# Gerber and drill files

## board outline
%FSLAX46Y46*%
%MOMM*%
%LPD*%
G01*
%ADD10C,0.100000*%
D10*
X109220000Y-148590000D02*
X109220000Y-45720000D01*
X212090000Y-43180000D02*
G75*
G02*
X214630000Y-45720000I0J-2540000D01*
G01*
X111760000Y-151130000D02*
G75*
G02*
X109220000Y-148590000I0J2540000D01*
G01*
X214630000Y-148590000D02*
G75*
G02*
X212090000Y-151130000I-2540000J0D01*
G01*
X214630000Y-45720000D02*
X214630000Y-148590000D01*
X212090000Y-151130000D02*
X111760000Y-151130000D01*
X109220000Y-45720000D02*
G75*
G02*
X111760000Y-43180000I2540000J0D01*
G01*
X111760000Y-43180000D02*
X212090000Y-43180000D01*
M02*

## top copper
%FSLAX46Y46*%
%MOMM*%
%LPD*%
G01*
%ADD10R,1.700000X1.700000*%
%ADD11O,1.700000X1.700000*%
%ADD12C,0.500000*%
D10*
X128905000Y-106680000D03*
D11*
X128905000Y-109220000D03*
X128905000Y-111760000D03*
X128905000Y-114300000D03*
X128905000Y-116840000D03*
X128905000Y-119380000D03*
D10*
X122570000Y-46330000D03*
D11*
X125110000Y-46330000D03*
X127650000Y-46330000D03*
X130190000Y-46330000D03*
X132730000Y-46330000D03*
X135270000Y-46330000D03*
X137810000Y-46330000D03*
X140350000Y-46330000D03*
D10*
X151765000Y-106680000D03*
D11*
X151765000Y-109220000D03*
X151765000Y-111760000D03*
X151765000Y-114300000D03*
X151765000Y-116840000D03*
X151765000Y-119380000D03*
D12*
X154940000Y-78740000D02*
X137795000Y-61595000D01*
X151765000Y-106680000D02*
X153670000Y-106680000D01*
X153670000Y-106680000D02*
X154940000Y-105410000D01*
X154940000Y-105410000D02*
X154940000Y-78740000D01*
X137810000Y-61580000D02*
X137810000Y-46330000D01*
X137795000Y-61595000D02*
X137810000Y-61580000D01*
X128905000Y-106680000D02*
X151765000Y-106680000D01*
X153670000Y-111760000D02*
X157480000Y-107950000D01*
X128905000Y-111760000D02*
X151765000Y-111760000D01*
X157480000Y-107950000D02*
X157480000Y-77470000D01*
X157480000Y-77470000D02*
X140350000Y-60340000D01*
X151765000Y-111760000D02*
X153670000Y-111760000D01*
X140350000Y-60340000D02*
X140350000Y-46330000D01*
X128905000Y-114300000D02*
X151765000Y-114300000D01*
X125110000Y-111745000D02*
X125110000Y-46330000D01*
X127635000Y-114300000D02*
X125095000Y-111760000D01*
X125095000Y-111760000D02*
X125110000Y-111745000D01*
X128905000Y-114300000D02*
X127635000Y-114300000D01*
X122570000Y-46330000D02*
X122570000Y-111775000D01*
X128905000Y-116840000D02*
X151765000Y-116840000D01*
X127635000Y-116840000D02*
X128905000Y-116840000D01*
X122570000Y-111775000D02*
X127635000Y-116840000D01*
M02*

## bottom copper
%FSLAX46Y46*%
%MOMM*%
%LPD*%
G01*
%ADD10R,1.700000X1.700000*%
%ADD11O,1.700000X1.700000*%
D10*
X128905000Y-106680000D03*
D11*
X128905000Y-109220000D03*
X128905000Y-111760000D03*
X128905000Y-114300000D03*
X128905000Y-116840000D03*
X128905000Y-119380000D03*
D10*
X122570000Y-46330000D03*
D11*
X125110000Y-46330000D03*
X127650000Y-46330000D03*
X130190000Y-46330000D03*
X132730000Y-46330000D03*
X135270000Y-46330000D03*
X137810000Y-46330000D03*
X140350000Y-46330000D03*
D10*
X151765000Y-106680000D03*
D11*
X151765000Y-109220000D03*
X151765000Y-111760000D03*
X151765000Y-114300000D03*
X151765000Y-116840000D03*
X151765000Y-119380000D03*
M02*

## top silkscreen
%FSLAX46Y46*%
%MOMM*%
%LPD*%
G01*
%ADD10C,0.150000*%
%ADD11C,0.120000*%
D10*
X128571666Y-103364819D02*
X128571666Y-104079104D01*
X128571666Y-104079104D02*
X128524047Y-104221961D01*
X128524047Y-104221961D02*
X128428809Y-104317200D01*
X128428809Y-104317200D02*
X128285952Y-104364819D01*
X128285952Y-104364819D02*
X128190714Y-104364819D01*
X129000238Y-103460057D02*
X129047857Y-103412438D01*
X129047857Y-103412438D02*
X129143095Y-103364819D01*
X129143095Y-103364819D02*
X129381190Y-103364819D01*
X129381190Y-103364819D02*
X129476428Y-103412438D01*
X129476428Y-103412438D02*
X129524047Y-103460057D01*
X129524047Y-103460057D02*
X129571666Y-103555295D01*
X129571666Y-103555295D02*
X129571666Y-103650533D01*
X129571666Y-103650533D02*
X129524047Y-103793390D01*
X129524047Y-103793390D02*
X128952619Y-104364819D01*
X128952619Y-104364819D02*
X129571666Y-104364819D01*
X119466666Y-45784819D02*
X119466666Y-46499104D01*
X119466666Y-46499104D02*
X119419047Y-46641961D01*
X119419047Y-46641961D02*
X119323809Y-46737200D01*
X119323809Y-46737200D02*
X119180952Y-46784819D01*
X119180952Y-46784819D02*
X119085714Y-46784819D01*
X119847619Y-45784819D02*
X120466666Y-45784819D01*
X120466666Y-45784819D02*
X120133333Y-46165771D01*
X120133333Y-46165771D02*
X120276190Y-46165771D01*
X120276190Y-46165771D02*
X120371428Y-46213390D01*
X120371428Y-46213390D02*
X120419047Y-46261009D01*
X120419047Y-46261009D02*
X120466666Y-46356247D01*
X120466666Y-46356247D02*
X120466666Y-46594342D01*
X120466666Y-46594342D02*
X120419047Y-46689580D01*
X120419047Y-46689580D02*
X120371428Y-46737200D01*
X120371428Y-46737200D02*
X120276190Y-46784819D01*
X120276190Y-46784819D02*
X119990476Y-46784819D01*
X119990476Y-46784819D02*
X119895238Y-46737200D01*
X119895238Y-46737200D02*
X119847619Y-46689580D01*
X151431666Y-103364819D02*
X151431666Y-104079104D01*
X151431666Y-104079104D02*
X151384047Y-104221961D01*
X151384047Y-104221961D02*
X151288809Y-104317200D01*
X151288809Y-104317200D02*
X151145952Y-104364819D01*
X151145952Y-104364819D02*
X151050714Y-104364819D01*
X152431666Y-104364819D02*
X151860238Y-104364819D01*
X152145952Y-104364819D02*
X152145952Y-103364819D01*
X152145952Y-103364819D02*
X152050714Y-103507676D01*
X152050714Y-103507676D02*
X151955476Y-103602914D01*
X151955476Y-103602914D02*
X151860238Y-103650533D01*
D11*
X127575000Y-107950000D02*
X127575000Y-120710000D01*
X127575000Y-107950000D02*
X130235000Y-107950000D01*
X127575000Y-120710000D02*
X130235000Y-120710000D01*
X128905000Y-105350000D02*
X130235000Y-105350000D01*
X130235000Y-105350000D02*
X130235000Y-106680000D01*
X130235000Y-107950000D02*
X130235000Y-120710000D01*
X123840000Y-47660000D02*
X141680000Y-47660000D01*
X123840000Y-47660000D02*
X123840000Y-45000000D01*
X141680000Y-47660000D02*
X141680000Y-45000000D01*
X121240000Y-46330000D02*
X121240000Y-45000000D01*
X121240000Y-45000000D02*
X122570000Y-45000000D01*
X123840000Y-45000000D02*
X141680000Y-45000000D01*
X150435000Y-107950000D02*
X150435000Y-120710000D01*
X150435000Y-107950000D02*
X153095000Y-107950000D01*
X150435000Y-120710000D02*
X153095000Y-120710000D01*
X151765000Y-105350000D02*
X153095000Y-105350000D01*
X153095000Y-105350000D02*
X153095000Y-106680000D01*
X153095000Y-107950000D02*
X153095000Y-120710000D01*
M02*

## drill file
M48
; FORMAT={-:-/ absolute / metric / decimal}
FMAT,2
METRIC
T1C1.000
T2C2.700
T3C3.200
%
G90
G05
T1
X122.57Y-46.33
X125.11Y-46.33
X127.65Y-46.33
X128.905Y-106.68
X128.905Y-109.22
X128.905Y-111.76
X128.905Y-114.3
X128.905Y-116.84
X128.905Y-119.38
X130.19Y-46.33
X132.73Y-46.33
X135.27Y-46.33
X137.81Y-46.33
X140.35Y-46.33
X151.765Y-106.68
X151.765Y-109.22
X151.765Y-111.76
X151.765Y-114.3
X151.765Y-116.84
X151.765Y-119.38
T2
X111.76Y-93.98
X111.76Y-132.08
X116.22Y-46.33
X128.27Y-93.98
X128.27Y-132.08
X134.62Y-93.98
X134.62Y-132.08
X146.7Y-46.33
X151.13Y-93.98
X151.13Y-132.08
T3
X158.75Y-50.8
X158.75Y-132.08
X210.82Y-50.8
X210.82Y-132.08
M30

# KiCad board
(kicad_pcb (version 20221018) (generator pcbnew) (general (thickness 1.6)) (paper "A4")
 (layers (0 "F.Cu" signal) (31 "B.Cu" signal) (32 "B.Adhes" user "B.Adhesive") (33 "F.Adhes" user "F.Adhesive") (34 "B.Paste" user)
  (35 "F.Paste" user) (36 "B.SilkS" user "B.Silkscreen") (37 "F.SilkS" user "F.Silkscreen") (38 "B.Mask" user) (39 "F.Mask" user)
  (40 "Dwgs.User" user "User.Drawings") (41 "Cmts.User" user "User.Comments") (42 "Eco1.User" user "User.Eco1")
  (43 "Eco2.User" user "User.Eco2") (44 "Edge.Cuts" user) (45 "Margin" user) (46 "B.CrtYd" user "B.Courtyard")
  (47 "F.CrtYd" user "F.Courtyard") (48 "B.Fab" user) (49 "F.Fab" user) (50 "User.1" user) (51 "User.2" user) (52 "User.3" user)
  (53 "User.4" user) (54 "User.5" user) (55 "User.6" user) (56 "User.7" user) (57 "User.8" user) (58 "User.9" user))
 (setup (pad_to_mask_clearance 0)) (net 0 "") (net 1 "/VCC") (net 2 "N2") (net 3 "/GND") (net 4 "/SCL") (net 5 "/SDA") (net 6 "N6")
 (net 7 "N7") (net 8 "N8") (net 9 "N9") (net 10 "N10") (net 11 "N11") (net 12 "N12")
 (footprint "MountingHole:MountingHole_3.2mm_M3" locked (layer "F.Cu") (at 158.75 132.08)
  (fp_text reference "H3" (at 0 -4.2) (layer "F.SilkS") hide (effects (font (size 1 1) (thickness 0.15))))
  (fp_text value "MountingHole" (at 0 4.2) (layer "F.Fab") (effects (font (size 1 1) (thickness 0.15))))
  (pad "" np_thru_hole circle locked (at 0 0) (size 3.2 3.2) (drill 3.2) (layers "*.Cu" "*.Mask")))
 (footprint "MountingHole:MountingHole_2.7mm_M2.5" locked (layer "F.Cu") (at 146.7 46.33)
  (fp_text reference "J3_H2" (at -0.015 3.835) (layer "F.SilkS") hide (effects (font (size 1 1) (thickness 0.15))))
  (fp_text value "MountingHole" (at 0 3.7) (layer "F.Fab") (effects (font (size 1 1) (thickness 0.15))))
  (pad "" np_thru_hole circle locked (at 0 0) (size 2.7 2.7) (drill 2.7) (layers "*.Cu" "*.Mask")))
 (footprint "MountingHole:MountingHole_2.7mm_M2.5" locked (layer "F.Cu") (at 128.27 93.98)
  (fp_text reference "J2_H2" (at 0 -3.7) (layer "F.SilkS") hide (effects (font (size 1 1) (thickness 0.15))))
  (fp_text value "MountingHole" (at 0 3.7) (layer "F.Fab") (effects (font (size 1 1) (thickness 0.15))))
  (pad "" np_thru_hole circle locked (at 0 0) (size 2.7 2.7) (drill 2.7) (layers "*.Cu" "*.Mask")))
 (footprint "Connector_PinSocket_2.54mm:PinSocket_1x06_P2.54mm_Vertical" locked (layer "F.Cu") (at 128.905 106.68)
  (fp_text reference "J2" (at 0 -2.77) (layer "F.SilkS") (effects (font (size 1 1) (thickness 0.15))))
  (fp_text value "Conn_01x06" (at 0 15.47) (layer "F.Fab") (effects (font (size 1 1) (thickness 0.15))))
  (fp_line (start -1.33 1.27) (end -1.33 14.03) (stroke (width 0.12) (type solid)) (layer "F.SilkS"))
  (fp_line (start -1.33 1.27) (end 1.33 1.27) (stroke (width 0.12) (type solid)) (layer "F.SilkS"))
  (fp_line (start -1.33 14.03) (end 1.33 14.03) (stroke (width 0.12) (type solid)) (layer "F.SilkS"))
  (fp_line (start 0 -1.33) (end 1.33 -1.33) (stroke (width 0.12) (type solid)) (layer "F.SilkS"))
  (fp_line (start 1.33 -1.33) (end 1.33 0) (stroke (width 0.12) (type solid)) (layer "F.SilkS"))
  (fp_line (start 1.33 1.27) (end 1.33 14.03) (stroke (width 0.12) (type solid)) (layer "F.SilkS"))
  (pad "1" thru_hole rect locked (at 0 0) (size 1.7 1.7) (drill 1) (layers "*.Cu" "*.Mask") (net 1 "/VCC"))
  (pad "2" thru_hole oval locked (at 0 2.54) (size 1.7 1.7) (drill 1) (layers "*.Cu" "*.Mask") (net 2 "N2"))
  (pad "3" thru_hole oval locked (at 0 5.08) (size 1.7 1.7) (drill 1) (layers "*.Cu" "*.Mask") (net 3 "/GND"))
  (pad "4" thru_hole oval locked (at 0 7.62) (size 1.7 1.7) (drill 1) (layers "*.Cu" "*.Mask") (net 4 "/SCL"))
  (pad "5" thru_hole oval locked (at 0 10.16) (size 1.7 1.7) (drill 1) (layers "*.Cu" "*.Mask") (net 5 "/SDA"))
  (pad "6" thru_hole oval locked (at 0 12.7) (size 1.7 1.7) (drill 1) (layers "*.Cu" "*.Mask") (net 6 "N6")))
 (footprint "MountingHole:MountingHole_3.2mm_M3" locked (layer "F.Cu") (at 158.75 50.8)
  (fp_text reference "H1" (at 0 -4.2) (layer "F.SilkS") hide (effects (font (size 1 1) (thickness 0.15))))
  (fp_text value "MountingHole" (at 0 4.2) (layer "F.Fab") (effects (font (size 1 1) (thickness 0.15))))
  (pad "" np_thru_hole circle locked (at 0 0) (size 3.2 3.2) (drill 3.2) (layers "*.Cu" "*.Mask")))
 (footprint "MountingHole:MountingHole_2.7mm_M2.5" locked (layer "F.Cu") (at 134.62 132.08)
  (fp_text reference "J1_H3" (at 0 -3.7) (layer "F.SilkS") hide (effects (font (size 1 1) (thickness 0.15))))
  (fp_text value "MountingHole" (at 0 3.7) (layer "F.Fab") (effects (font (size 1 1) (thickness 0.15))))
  (pad "" np_thru_hole circle locked (at 0 0) (size 2.7 2.7) (drill 2.7) (layers "*.Cu" "*.Mask")))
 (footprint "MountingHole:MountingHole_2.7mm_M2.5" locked (layer "F.Cu") (at 116.22 46.33)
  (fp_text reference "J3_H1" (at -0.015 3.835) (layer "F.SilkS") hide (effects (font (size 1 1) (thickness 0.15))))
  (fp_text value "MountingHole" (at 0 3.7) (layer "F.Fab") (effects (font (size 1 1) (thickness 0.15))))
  (pad "" np_thru_hole circle locked (at 0 0) (size 2.7 2.7) (drill 2.7) (layers "*.Cu" "*.Mask")))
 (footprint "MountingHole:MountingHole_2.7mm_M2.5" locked (layer "F.Cu") (at 151.13 132.08)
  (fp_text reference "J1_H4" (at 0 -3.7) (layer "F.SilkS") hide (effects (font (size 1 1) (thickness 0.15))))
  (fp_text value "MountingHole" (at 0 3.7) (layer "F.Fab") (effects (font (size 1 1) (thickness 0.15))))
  (pad "" np_thru_hole circle locked (at 0 0) (size 2.7 2.7) (drill 2.7) (layers "*.Cu" "*.Mask")))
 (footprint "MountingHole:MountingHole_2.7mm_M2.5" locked (layer "F.Cu") (at 134.62 93.98)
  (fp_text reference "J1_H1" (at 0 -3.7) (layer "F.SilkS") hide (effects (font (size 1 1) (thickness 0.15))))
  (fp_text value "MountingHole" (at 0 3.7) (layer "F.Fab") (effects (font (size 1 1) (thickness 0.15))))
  (pad "" np_thru_hole circle locked (at 0 0) (size 2.7 2.7) (drill 2.7) (layers "*.Cu" "*.Mask")))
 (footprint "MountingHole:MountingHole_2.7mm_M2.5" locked (layer "F.Cu") (at 111.76 132.08)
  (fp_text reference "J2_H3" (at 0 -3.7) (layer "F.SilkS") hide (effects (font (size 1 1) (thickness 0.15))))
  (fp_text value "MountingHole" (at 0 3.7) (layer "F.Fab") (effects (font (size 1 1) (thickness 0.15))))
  (pad "" np_thru_hole circle locked (at 0 0) (size 2.7 2.7) (drill 2.7) (layers "*.Cu" "*.Mask")))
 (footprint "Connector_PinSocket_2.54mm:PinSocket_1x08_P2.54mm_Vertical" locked (layer "F.Cu") (at 122.57 46.33 90)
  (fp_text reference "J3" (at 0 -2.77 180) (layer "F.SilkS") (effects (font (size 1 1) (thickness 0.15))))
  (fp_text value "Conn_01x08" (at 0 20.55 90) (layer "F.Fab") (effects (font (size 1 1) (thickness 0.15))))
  (fp_line (start -1.33 1.27) (end -1.33 19.11) (stroke (width 0.12) (type solid)) (layer "F.SilkS"))
  (fp_line (start -1.33 1.27) (end 1.33 1.27) (stroke (width 0.12) (type solid)) (layer "F.SilkS"))
  (fp_line (start -1.33 19.11) (end 1.33 19.11) (stroke (width 0.12) (type solid)) (layer "F.SilkS"))
  (fp_line (start 0 -1.33) (end 1.33 -1.33) (stroke (width 0.12) (type solid)) (layer "F.SilkS"))
  (fp_line (start 1.33 -1.33) (end 1.33 0) (stroke (width 0.12) (type solid)) (layer "F.SilkS"))
  (fp_line (start 1.33 1.27) (end 1.33 19.11) (stroke (width 0.12) (type solid)) (layer "F.SilkS"))
  (pad "1" thru_hole rect locked (at 0 0 90) (size 1.7 1.7) (drill 1) (layers "*.Cu" "*.Mask") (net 5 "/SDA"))
  (pad "2" thru_hole oval locked (at 0 2.54 90) (size 1.7 1.7) (drill 1) (layers "*.Cu" "*.Mask") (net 4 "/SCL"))
  (pad "3" thru_hole oval locked (at 0 5.08 90) (size 1.7 1.7) (drill 1) (layers "*.Cu" "*.Mask") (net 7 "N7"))
  (pad "4" thru_hole oval locked (at 0 7.62 90) (size 1.7 1.7) (drill 1) (layers "*.Cu" "*.Mask") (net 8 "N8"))
  (pad "5" thru_hole oval locked (at 0 10.16 90) (size 1.7 1.7) (drill 1) (layers "*.Cu" "*.Mask") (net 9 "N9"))
  (pad "6" thru_hole oval locked (at 0 12.7 90) (size 1.7 1.7) (drill 1) (layers "*.Cu" "*.Mask") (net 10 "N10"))
  (pad "7" thru_hole oval locked (at 0 15.24 90) (size 1.7 1.7) (drill 1) (layers "*.Cu" "*.Mask") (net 1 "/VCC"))
  (pad "8" thru_hole oval locked (at 0 17.78 90) (size 1.7 1.7) (drill 1) (layers "*.Cu" "*.Mask") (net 3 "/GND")))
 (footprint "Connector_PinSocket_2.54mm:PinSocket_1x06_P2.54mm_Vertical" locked (layer "F.Cu") (at 151.765 106.68)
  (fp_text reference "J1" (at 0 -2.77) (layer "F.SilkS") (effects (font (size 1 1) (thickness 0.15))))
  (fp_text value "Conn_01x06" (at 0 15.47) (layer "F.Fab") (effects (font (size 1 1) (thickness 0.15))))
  (fp_line (start -1.33 1.27) (end -1.33 14.03) (stroke (width 0.12) (type solid)) (layer "F.SilkS"))
  (fp_line (start -1.33 1.27) (end 1.33 1.27) (stroke (width 0.12) (type solid)) (layer "F.SilkS"))
  (fp_line (start -1.33 14.03) (end 1.33 14.03) (stroke (width 0.12) (type solid)) (layer "F.SilkS"))
  (fp_line (start 0 -1.33) (end 1.33 -1.33) (stroke (width 0.12) (type solid)) (layer "F.SilkS"))
  (fp_line (start 1.33 -1.33) (end 1.33 0) (stroke (width 0.12) (type solid)) (layer "F.SilkS"))
  (fp_line (start 1.33 1.27) (end 1.33 14.03) (stroke (width 0.12) (type solid)) (layer "F.SilkS"))
  (pad "1" thru_hole rect locked (at 0 0) (size 1.7 1.7) (drill 1) (layers "*.Cu" "*.Mask") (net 1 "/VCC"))
  (pad "2" thru_hole oval locked (at 0 2.54) (size 1.7 1.7) (drill 1) (layers "*.Cu" "*.Mask") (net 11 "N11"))
  (pad "3" thru_hole oval locked (at 0 5.08) (size 1.7 1.7) (drill 1) (layers "*.Cu" "*.Mask") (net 3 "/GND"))
  (pad "4" thru_hole oval locked (at 0 7.62) (size 1.7 1.7) (drill 1) (layers "*.Cu" "*.Mask") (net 4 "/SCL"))
  (pad "5" thru_hole oval locked (at 0 10.16) (size 1.7 1.7) (drill 1) (layers "*.Cu" "*.Mask") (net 5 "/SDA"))
  (pad "6" thru_hole oval locked (at 0 12.7) (size 1.7 1.7) (drill 1) (layers "*.Cu" "*.Mask") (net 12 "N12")))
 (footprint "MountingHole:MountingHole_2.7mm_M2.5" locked (layer "F.Cu") (at 151.13 93.98)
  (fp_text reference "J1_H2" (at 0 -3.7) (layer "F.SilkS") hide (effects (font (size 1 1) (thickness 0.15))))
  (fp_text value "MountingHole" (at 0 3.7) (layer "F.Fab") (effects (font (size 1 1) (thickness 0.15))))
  (pad "" np_thru_hole circle locked (at 0 0) (size 2.7 2.7) (drill 2.7) (layers "*.Cu" "*.Mask")))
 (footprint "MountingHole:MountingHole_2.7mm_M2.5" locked (layer "F.Cu") (at 128.27 132.08)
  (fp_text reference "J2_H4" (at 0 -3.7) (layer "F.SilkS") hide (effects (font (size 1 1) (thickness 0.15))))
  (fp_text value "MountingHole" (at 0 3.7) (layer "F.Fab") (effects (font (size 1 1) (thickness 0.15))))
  (pad "" np_thru_hole circle locked (at 0 0) (size 2.7 2.7) (drill 2.7) (layers "*.Cu" "*.Mask")))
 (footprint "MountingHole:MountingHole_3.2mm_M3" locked (layer "F.Cu") (at 210.82 50.8)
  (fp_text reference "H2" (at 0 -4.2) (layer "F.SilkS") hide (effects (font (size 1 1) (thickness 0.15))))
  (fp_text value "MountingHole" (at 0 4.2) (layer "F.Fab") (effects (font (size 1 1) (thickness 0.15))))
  (pad "" np_thru_hole circle locked (at 0 0) (size 3.2 3.2) (drill 3.2) (layers "*.Cu" "*.Mask")))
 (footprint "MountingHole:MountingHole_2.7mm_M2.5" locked (layer "F.Cu") (at 111.76 93.98)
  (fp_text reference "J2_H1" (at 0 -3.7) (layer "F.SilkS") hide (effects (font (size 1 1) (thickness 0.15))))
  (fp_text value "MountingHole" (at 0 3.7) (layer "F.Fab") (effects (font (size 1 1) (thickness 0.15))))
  (pad "" np_thru_hole circle locked (at 0 0) (size 2.7 2.7) (drill 2.7) (layers "*.Cu" "*.Mask")))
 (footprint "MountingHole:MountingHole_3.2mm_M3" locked (layer "F.Cu") (at 210.82 132.08)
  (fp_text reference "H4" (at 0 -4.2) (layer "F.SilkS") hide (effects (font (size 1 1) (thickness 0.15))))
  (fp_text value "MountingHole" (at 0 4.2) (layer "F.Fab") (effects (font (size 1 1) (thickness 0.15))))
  (pad "" np_thru_hole circle locked (at 0 0) (size 3.2 3.2) (drill 3.2) (layers "*.Cu" "*.Mask")))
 (gr_line (start 109.22 148.59) (end 109.22 45.72) (stroke (width 0.1) (type default)) (layer "Edge.Cuts"))
 (gr_arc (start 212.09 43.18) (mid 213.886051 43.923949) (end 214.63 45.72) (stroke (width 0.1) (type default)) (layer "Edge.Cuts"))
 (gr_arc (start 111.76 151.13) (mid 109.963949 150.386051) (end 109.22 148.59) (stroke (width 0.1) (type default)) (layer "Edge.Cuts"))
 (gr_arc (start 214.63 148.59) (mid 213.886051 150.386051) (end 212.09 151.13) (stroke (width 0.1) (type default)) (layer "Edge.Cuts"))
 (gr_line (start 214.63 45.72) (end 214.63 148.59) (stroke (width 0.1) (type default)) (layer "Edge.Cuts"))
 (gr_line (start 212.09 151.13) (end 111.76 151.13) (stroke (width 0.1) (type default)) (layer "Edge.Cuts"))
 (gr_arc (start 109.22 45.72) (mid 109.963949 43.923949) (end 111.76 43.18) (stroke (width 0.1) (type default)) (layer "Edge.Cuts"))
 (gr_line (start 111.76 43.18) (end 212.09 43.18) (stroke (width 0.1) (type default)) (layer "Edge.Cuts"))
 (segment (start 154.94 78.74) (end 137.795 61.595) (width 0.5) (layer "F.Cu") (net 1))
 (segment (start 151.765 106.68) (end 153.67 106.68) (width 0.5) (layer "F.Cu") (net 1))
 (segment (start 153.67 106.68) (end 154.94 105.41) (width 0.5) (layer "F.Cu") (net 1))
 (segment (start 154.94 105.41) (end 154.94 78.74) (width 0.5) (layer "F.Cu") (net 1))
 (segment (start 137.81 61.58) (end 137.81 46.33) (width 0.5) (layer "F.Cu") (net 1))
 (segment (start 137.795 61.595) (end 137.81 61.58) (width 0.5) (layer "F.Cu") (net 1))
 (segment (start 128.905 106.68) (end 151.765 106.68) (width 0.5) (layer "F.Cu") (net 1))
 (segment (start 153.67 111.76) (end 157.48 107.95) (width 0.5) (layer "F.Cu") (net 3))
 (segment (start 128.905 111.76) (end 151.765 111.76) (width 0.5) (layer "F.Cu") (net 3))
 (segment (start 157.48 107.95) (end 157.48 77.47) (width 0.5) (layer "F.Cu") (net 3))
 (segment (start 157.48 77.47) (end 140.35 60.34) (width 0.5) (layer "F.Cu") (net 3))
 (segment (start 151.765 111.76) (end 153.67 111.76) (width 0.5) (layer "F.Cu") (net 3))
 (segment (start 140.35 60.34) (end 140.35 46.33) (width 0.5) (layer "F.Cu") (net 3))
 (segment (start 128.905 114.3) (end 151.765 114.3) (width 0.5) (layer "F.Cu") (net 4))
 (segment (start 125.11 111.745) (end 125.11 46.33) (width 0.5) (layer "F.Cu") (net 4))
 (segment (start 127.635 114.3) (end 125.095 111.76) (width 0.5) (layer "F.Cu") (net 4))
 (segment (start 125.095 111.76) (end 125.11 111.745) (width 0.5) (layer "F.Cu") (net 4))
 (segment (start 128.905 114.3) (end 127.635 114.3) (width 0.5) (layer "F.Cu") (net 4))
 (segment (start 122.57 46.33) (end 122.57 111.775) (width 0.5) (layer "F.Cu") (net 5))
 (segment (start 128.905 116.84) (end 151.765 116.84) (width 0.5) (layer "F.Cu") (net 5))
 (segment (start 127.635 116.84) (end 128.905 116.84) (width 0.5) (layer "F.Cu") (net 5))
 (segment (start 122.57 111.775) (end 127.635 116.84) (width 0.5) (layer "F.Cu") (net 5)))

